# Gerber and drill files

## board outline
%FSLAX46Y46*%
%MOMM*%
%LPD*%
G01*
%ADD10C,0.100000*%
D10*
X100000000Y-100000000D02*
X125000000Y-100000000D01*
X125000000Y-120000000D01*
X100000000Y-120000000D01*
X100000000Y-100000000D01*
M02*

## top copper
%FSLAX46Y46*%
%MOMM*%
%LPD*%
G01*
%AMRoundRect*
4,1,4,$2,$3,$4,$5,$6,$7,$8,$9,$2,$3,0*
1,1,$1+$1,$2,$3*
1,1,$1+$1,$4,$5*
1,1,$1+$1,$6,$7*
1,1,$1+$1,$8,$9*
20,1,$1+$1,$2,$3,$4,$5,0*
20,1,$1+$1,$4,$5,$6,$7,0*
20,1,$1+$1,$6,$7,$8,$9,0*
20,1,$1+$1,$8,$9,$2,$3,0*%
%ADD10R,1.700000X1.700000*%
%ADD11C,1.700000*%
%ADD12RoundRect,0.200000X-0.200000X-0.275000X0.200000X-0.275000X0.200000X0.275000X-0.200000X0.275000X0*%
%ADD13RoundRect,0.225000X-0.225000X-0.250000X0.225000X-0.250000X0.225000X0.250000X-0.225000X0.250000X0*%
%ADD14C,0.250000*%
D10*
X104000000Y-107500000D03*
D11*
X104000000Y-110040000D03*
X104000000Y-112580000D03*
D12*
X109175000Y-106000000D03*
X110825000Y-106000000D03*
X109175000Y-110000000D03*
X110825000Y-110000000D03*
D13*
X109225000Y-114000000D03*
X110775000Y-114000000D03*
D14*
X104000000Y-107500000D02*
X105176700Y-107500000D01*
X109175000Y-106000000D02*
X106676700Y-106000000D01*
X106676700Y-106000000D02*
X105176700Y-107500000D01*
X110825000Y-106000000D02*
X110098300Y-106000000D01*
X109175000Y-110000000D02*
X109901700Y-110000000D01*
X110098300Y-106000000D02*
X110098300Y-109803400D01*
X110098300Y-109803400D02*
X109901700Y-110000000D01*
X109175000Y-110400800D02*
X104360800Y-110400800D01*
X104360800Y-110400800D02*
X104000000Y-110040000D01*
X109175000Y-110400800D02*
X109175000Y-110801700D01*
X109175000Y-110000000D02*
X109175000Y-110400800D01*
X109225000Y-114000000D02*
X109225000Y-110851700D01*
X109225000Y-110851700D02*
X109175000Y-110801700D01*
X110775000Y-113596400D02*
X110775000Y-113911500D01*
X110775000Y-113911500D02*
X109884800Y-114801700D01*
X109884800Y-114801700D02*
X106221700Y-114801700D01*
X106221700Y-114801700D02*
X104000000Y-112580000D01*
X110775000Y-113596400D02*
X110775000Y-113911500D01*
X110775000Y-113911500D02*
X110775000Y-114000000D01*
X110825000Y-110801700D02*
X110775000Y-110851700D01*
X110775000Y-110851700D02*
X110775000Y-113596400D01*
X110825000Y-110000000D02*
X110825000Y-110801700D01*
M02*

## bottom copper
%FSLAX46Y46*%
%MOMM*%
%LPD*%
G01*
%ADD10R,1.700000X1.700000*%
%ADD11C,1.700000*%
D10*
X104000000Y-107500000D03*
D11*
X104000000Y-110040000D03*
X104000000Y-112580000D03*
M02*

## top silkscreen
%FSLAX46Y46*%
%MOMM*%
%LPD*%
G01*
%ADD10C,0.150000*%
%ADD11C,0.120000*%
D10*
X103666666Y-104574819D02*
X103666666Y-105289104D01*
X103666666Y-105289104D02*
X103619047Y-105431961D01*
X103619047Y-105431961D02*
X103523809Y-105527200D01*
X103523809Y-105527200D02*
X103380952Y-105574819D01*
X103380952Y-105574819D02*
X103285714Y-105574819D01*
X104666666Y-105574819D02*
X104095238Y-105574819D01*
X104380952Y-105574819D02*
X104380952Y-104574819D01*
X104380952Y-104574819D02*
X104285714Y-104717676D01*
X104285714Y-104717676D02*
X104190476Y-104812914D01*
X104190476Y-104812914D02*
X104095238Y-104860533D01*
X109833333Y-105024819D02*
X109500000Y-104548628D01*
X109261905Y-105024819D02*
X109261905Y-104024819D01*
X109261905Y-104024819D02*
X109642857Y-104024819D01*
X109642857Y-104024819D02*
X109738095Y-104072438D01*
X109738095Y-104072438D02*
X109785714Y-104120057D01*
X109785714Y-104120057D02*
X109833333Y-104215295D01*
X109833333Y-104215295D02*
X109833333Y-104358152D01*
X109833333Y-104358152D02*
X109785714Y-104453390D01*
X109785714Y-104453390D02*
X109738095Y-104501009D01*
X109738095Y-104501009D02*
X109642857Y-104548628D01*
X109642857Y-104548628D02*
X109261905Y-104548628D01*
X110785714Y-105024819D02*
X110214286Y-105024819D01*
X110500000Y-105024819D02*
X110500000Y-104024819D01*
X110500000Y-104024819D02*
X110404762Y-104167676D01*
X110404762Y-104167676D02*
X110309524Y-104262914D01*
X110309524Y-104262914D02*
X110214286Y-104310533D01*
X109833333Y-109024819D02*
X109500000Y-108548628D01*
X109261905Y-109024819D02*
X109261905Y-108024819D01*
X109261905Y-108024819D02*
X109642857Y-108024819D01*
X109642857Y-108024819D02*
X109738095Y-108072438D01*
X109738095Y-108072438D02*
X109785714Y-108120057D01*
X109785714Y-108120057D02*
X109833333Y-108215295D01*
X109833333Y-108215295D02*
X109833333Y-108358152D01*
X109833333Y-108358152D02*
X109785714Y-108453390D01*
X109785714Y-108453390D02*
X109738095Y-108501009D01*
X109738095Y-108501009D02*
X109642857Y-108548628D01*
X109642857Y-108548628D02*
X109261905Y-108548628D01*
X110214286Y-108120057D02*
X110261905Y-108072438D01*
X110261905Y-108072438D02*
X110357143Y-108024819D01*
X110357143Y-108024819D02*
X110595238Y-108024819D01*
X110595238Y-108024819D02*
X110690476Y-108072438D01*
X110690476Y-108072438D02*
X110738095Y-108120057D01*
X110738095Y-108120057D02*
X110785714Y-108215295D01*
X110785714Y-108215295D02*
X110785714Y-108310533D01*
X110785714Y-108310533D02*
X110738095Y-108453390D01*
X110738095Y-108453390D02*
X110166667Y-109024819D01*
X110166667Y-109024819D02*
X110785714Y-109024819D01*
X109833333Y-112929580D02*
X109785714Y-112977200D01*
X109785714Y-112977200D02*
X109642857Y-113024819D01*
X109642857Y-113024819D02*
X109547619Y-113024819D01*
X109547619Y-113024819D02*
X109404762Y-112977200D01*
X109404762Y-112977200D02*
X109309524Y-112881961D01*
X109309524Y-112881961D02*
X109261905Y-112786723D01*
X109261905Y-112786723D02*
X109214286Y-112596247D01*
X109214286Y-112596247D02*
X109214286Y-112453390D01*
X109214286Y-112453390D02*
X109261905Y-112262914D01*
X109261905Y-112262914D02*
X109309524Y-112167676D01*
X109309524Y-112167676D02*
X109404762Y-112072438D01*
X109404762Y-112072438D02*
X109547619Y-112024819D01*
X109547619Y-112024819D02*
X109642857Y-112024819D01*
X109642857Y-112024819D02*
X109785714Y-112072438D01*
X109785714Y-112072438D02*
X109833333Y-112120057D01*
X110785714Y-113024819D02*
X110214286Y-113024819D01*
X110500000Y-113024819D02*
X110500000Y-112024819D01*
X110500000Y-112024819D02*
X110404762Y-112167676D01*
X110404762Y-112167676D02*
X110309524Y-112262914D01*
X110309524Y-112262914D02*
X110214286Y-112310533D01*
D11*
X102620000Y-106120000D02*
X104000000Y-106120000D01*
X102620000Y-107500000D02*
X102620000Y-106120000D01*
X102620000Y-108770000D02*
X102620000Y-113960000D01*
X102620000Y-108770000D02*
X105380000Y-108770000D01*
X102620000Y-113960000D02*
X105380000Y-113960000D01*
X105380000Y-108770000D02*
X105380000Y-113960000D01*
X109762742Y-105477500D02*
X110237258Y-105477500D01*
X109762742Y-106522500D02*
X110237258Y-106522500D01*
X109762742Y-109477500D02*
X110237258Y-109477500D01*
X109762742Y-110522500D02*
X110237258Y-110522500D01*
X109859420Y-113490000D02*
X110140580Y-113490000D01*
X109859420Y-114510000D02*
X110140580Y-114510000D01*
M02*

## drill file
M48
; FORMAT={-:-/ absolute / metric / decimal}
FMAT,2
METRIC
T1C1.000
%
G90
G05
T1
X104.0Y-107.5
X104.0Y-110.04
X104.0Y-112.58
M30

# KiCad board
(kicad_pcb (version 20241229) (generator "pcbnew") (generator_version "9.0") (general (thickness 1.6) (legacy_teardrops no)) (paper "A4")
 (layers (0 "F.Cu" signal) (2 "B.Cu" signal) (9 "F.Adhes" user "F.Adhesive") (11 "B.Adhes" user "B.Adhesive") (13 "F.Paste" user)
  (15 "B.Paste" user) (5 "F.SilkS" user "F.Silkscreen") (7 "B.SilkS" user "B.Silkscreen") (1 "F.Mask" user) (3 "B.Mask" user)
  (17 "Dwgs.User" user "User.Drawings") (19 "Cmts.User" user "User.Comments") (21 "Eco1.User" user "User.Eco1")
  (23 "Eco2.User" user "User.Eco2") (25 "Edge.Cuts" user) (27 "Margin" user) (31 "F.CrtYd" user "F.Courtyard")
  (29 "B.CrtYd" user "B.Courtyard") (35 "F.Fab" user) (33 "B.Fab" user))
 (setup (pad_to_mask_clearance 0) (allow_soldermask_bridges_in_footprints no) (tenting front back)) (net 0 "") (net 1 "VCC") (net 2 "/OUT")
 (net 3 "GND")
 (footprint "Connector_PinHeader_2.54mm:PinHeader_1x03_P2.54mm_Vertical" (layer "F.Cu") (at 104 107.5)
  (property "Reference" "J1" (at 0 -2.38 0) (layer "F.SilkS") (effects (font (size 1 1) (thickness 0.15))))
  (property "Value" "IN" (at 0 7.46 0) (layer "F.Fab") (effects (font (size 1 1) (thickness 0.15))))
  (fp_line (start -1.38 -1.38) (end 0 -1.38) (stroke (width 0.12) (type solid)) (layer "F.SilkS"))
  (fp_line (start -1.38 0) (end -1.38 -1.38) (stroke (width 0.12) (type solid)) (layer "F.SilkS"))
  (fp_line (start -1.38 1.27) (end -1.38 6.46) (stroke (width 0.12) (type solid)) (layer "F.SilkS"))
  (fp_line (start -1.38 1.27) (end 1.38 1.27) (stroke (width 0.12) (type solid)) (layer "F.SilkS"))
  (fp_line (start -1.38 6.46) (end 1.38 6.46) (stroke (width 0.12) (type solid)) (layer "F.SilkS"))
  (fp_line (start 1.38 1.27) (end 1.38 6.46) (stroke (width 0.12) (type solid)) (layer "F.SilkS"))
  (pad "1" thru_hole rect (at 0 0) (size 1.7 1.7) (drill 1) (layers "*.Cu" "*.Mask") (remove_unused_layers no) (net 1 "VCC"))
  (pad "2" thru_hole circle (at 0 2.54) (size 1.7 1.7) (drill 1) (layers "*.Cu" "*.Mask") (remove_unused_layers no) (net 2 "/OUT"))
  (pad "3" thru_hole circle (at 0 5.08) (size 1.7 1.7) (drill 1) (layers "*.Cu" "*.Mask") (remove_unused_layers no) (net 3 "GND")))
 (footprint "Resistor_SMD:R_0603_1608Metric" (layer "F.Cu") (at 110 106)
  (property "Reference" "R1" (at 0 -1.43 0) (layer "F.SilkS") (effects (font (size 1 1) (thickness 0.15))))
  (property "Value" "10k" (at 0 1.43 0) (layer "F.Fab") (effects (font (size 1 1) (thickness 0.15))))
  (fp_line (start -0.237258 -0.5225) (end 0.237258 -0.5225) (stroke (width 0.12) (type solid)) (layer "F.SilkS"))
  (fp_line (start -0.237258 0.5225) (end 0.237258 0.5225) (stroke (width 0.12) (type solid)) (layer "F.SilkS"))
  (pad "1" smd roundrect (at -0.825 0) (size 0.8 0.95) (layers "F.Cu" "F.Mask" "F.Paste") (roundrect_rratio 0.25) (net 1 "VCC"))
  (pad "2" smd roundrect (at 0.825 0) (size 0.8 0.95) (layers "F.Cu" "F.Mask" "F.Paste") (roundrect_rratio 0.25) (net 2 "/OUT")))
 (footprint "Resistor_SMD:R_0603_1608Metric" (layer "F.Cu") (at 110 110)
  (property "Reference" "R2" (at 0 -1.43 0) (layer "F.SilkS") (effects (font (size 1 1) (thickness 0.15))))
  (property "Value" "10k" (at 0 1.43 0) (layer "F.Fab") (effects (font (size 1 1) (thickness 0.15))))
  (fp_line (start -0.237258 -0.5225) (end 0.237258 -0.5225) (stroke (width 0.12) (type solid)) (layer "F.SilkS"))
  (fp_line (start -0.237258 0.5225) (end 0.237258 0.5225) (stroke (width 0.12) (type solid)) (layer "F.SilkS"))
  (pad "1" smd roundrect (at -0.825 0) (size 0.8 0.95) (layers "F.Cu" "F.Mask" "F.Paste") (roundrect_rratio 0.25) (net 2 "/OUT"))
  (pad "2" smd roundrect (at 0.825 0) (size 0.8 0.95) (layers "F.Cu" "F.Mask" "F.Paste") (roundrect_rratio 0.25) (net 3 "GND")))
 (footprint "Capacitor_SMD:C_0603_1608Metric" (layer "F.Cu") (at 110 114)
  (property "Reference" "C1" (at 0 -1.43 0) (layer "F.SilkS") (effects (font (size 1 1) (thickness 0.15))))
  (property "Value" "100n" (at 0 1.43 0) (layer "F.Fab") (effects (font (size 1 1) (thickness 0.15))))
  (fp_line (start -0.14058 -0.51) (end 0.14058 -0.51) (stroke (width 0.12) (type solid)) (layer "F.SilkS"))
  (fp_line (start -0.14058 0.51) (end 0.14058 0.51) (stroke (width 0.12) (type solid)) (layer "F.SilkS"))
  (pad "1" smd roundrect (at -0.775 0) (size 0.9 0.95) (layers "F.Cu" "F.Mask" "F.Paste") (roundrect_rratio 0.25) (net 2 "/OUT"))
  (pad "2" smd roundrect (at 0.775 0) (size 0.9 0.95) (layers "F.Cu" "F.Mask" "F.Paste") (roundrect_rratio 0.25) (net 3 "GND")))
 (gr_rect (start 100 100) (end 125 120) (stroke (width 0.1) (type default)) (fill no) (layer "Edge.Cuts"))
 (segment (start 104 107.5) (end 105.1767 107.5) (width 0.25) (layer "F.Cu") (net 1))
 (segment (start 109.175 106) (end 106.6767 106) (width 0.25) (layer "F.Cu") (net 1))
 (segment (start 106.6767 106) (end 105.1767 107.5) (width 0.25) (layer "F.Cu") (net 1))
 (segment (start 110.825 106) (end 110.0983 106) (width 0.25) (layer "F.Cu") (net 2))
 (segment (start 109.175 110) (end 109.9017 110) (width 0.25) (layer "F.Cu") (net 2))
 (segment (start 110.0983 106) (end 110.0983 109.8034) (width 0.25) (layer "F.Cu") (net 2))
 (segment (start 110.0983 109.8034) (end 109.9017 110) (width 0.25) (layer "F.Cu") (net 2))
 (segment (start 109.175 110.4008) (end 104.3608 110.4008) (width 0.25) (layer "F.Cu") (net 2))
 (segment (start 104.3608 110.4008) (end 104 110.04) (width 0.25) (layer "F.Cu") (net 2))
 (segment (start 109.175 110.4008) (end 109.175 110.8017) (width 0.25) (layer "F.Cu") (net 2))
 (segment (start 109.175 110) (end 109.175 110.4008) (width 0.25) (layer "F.Cu") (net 2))
 (segment (start 109.225 114) (end 109.225 110.8517) (width 0.25) (layer "F.Cu") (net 2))
 (segment (start 109.225 110.8517) (end 109.175 110.8017) (width 0.25) (layer "F.Cu") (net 2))
 (segment (start 110.775 113.5964) (end 110.775 113.9115) (width 0.25) (layer "F.Cu") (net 3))
 (segment (start 110.775 113.9115) (end 109.8848 114.8017) (width 0.25) (layer "F.Cu") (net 3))
 (segment (start 109.8848 114.8017) (end 106.2217 114.8017) (width 0.25) (layer "F.Cu") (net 3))
 (segment (start 106.2217 114.8017) (end 104 112.58) (width 0.25) (layer "F.Cu") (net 3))
 (segment (start 110.775 113.5964) (end 110.775 113.9115) (width 0.25) (layer "F.Cu") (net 3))
 (segment (start 110.775 113.9115) (end 110.775 114) (width 0.25) (layer "F.Cu") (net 3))
 (segment (start 110.825 110.8017) (end 110.775 110.8517) (width 0.25) (layer "F.Cu") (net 3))
 (segment (start 110.775 110.8517) (end 110.775 113.5964) (width 0.25) (layer "F.Cu") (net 3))
 (segment (start 110.825 110) (end 110.825 110.8017) (width 0.25) (layer "F.Cu") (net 3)))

